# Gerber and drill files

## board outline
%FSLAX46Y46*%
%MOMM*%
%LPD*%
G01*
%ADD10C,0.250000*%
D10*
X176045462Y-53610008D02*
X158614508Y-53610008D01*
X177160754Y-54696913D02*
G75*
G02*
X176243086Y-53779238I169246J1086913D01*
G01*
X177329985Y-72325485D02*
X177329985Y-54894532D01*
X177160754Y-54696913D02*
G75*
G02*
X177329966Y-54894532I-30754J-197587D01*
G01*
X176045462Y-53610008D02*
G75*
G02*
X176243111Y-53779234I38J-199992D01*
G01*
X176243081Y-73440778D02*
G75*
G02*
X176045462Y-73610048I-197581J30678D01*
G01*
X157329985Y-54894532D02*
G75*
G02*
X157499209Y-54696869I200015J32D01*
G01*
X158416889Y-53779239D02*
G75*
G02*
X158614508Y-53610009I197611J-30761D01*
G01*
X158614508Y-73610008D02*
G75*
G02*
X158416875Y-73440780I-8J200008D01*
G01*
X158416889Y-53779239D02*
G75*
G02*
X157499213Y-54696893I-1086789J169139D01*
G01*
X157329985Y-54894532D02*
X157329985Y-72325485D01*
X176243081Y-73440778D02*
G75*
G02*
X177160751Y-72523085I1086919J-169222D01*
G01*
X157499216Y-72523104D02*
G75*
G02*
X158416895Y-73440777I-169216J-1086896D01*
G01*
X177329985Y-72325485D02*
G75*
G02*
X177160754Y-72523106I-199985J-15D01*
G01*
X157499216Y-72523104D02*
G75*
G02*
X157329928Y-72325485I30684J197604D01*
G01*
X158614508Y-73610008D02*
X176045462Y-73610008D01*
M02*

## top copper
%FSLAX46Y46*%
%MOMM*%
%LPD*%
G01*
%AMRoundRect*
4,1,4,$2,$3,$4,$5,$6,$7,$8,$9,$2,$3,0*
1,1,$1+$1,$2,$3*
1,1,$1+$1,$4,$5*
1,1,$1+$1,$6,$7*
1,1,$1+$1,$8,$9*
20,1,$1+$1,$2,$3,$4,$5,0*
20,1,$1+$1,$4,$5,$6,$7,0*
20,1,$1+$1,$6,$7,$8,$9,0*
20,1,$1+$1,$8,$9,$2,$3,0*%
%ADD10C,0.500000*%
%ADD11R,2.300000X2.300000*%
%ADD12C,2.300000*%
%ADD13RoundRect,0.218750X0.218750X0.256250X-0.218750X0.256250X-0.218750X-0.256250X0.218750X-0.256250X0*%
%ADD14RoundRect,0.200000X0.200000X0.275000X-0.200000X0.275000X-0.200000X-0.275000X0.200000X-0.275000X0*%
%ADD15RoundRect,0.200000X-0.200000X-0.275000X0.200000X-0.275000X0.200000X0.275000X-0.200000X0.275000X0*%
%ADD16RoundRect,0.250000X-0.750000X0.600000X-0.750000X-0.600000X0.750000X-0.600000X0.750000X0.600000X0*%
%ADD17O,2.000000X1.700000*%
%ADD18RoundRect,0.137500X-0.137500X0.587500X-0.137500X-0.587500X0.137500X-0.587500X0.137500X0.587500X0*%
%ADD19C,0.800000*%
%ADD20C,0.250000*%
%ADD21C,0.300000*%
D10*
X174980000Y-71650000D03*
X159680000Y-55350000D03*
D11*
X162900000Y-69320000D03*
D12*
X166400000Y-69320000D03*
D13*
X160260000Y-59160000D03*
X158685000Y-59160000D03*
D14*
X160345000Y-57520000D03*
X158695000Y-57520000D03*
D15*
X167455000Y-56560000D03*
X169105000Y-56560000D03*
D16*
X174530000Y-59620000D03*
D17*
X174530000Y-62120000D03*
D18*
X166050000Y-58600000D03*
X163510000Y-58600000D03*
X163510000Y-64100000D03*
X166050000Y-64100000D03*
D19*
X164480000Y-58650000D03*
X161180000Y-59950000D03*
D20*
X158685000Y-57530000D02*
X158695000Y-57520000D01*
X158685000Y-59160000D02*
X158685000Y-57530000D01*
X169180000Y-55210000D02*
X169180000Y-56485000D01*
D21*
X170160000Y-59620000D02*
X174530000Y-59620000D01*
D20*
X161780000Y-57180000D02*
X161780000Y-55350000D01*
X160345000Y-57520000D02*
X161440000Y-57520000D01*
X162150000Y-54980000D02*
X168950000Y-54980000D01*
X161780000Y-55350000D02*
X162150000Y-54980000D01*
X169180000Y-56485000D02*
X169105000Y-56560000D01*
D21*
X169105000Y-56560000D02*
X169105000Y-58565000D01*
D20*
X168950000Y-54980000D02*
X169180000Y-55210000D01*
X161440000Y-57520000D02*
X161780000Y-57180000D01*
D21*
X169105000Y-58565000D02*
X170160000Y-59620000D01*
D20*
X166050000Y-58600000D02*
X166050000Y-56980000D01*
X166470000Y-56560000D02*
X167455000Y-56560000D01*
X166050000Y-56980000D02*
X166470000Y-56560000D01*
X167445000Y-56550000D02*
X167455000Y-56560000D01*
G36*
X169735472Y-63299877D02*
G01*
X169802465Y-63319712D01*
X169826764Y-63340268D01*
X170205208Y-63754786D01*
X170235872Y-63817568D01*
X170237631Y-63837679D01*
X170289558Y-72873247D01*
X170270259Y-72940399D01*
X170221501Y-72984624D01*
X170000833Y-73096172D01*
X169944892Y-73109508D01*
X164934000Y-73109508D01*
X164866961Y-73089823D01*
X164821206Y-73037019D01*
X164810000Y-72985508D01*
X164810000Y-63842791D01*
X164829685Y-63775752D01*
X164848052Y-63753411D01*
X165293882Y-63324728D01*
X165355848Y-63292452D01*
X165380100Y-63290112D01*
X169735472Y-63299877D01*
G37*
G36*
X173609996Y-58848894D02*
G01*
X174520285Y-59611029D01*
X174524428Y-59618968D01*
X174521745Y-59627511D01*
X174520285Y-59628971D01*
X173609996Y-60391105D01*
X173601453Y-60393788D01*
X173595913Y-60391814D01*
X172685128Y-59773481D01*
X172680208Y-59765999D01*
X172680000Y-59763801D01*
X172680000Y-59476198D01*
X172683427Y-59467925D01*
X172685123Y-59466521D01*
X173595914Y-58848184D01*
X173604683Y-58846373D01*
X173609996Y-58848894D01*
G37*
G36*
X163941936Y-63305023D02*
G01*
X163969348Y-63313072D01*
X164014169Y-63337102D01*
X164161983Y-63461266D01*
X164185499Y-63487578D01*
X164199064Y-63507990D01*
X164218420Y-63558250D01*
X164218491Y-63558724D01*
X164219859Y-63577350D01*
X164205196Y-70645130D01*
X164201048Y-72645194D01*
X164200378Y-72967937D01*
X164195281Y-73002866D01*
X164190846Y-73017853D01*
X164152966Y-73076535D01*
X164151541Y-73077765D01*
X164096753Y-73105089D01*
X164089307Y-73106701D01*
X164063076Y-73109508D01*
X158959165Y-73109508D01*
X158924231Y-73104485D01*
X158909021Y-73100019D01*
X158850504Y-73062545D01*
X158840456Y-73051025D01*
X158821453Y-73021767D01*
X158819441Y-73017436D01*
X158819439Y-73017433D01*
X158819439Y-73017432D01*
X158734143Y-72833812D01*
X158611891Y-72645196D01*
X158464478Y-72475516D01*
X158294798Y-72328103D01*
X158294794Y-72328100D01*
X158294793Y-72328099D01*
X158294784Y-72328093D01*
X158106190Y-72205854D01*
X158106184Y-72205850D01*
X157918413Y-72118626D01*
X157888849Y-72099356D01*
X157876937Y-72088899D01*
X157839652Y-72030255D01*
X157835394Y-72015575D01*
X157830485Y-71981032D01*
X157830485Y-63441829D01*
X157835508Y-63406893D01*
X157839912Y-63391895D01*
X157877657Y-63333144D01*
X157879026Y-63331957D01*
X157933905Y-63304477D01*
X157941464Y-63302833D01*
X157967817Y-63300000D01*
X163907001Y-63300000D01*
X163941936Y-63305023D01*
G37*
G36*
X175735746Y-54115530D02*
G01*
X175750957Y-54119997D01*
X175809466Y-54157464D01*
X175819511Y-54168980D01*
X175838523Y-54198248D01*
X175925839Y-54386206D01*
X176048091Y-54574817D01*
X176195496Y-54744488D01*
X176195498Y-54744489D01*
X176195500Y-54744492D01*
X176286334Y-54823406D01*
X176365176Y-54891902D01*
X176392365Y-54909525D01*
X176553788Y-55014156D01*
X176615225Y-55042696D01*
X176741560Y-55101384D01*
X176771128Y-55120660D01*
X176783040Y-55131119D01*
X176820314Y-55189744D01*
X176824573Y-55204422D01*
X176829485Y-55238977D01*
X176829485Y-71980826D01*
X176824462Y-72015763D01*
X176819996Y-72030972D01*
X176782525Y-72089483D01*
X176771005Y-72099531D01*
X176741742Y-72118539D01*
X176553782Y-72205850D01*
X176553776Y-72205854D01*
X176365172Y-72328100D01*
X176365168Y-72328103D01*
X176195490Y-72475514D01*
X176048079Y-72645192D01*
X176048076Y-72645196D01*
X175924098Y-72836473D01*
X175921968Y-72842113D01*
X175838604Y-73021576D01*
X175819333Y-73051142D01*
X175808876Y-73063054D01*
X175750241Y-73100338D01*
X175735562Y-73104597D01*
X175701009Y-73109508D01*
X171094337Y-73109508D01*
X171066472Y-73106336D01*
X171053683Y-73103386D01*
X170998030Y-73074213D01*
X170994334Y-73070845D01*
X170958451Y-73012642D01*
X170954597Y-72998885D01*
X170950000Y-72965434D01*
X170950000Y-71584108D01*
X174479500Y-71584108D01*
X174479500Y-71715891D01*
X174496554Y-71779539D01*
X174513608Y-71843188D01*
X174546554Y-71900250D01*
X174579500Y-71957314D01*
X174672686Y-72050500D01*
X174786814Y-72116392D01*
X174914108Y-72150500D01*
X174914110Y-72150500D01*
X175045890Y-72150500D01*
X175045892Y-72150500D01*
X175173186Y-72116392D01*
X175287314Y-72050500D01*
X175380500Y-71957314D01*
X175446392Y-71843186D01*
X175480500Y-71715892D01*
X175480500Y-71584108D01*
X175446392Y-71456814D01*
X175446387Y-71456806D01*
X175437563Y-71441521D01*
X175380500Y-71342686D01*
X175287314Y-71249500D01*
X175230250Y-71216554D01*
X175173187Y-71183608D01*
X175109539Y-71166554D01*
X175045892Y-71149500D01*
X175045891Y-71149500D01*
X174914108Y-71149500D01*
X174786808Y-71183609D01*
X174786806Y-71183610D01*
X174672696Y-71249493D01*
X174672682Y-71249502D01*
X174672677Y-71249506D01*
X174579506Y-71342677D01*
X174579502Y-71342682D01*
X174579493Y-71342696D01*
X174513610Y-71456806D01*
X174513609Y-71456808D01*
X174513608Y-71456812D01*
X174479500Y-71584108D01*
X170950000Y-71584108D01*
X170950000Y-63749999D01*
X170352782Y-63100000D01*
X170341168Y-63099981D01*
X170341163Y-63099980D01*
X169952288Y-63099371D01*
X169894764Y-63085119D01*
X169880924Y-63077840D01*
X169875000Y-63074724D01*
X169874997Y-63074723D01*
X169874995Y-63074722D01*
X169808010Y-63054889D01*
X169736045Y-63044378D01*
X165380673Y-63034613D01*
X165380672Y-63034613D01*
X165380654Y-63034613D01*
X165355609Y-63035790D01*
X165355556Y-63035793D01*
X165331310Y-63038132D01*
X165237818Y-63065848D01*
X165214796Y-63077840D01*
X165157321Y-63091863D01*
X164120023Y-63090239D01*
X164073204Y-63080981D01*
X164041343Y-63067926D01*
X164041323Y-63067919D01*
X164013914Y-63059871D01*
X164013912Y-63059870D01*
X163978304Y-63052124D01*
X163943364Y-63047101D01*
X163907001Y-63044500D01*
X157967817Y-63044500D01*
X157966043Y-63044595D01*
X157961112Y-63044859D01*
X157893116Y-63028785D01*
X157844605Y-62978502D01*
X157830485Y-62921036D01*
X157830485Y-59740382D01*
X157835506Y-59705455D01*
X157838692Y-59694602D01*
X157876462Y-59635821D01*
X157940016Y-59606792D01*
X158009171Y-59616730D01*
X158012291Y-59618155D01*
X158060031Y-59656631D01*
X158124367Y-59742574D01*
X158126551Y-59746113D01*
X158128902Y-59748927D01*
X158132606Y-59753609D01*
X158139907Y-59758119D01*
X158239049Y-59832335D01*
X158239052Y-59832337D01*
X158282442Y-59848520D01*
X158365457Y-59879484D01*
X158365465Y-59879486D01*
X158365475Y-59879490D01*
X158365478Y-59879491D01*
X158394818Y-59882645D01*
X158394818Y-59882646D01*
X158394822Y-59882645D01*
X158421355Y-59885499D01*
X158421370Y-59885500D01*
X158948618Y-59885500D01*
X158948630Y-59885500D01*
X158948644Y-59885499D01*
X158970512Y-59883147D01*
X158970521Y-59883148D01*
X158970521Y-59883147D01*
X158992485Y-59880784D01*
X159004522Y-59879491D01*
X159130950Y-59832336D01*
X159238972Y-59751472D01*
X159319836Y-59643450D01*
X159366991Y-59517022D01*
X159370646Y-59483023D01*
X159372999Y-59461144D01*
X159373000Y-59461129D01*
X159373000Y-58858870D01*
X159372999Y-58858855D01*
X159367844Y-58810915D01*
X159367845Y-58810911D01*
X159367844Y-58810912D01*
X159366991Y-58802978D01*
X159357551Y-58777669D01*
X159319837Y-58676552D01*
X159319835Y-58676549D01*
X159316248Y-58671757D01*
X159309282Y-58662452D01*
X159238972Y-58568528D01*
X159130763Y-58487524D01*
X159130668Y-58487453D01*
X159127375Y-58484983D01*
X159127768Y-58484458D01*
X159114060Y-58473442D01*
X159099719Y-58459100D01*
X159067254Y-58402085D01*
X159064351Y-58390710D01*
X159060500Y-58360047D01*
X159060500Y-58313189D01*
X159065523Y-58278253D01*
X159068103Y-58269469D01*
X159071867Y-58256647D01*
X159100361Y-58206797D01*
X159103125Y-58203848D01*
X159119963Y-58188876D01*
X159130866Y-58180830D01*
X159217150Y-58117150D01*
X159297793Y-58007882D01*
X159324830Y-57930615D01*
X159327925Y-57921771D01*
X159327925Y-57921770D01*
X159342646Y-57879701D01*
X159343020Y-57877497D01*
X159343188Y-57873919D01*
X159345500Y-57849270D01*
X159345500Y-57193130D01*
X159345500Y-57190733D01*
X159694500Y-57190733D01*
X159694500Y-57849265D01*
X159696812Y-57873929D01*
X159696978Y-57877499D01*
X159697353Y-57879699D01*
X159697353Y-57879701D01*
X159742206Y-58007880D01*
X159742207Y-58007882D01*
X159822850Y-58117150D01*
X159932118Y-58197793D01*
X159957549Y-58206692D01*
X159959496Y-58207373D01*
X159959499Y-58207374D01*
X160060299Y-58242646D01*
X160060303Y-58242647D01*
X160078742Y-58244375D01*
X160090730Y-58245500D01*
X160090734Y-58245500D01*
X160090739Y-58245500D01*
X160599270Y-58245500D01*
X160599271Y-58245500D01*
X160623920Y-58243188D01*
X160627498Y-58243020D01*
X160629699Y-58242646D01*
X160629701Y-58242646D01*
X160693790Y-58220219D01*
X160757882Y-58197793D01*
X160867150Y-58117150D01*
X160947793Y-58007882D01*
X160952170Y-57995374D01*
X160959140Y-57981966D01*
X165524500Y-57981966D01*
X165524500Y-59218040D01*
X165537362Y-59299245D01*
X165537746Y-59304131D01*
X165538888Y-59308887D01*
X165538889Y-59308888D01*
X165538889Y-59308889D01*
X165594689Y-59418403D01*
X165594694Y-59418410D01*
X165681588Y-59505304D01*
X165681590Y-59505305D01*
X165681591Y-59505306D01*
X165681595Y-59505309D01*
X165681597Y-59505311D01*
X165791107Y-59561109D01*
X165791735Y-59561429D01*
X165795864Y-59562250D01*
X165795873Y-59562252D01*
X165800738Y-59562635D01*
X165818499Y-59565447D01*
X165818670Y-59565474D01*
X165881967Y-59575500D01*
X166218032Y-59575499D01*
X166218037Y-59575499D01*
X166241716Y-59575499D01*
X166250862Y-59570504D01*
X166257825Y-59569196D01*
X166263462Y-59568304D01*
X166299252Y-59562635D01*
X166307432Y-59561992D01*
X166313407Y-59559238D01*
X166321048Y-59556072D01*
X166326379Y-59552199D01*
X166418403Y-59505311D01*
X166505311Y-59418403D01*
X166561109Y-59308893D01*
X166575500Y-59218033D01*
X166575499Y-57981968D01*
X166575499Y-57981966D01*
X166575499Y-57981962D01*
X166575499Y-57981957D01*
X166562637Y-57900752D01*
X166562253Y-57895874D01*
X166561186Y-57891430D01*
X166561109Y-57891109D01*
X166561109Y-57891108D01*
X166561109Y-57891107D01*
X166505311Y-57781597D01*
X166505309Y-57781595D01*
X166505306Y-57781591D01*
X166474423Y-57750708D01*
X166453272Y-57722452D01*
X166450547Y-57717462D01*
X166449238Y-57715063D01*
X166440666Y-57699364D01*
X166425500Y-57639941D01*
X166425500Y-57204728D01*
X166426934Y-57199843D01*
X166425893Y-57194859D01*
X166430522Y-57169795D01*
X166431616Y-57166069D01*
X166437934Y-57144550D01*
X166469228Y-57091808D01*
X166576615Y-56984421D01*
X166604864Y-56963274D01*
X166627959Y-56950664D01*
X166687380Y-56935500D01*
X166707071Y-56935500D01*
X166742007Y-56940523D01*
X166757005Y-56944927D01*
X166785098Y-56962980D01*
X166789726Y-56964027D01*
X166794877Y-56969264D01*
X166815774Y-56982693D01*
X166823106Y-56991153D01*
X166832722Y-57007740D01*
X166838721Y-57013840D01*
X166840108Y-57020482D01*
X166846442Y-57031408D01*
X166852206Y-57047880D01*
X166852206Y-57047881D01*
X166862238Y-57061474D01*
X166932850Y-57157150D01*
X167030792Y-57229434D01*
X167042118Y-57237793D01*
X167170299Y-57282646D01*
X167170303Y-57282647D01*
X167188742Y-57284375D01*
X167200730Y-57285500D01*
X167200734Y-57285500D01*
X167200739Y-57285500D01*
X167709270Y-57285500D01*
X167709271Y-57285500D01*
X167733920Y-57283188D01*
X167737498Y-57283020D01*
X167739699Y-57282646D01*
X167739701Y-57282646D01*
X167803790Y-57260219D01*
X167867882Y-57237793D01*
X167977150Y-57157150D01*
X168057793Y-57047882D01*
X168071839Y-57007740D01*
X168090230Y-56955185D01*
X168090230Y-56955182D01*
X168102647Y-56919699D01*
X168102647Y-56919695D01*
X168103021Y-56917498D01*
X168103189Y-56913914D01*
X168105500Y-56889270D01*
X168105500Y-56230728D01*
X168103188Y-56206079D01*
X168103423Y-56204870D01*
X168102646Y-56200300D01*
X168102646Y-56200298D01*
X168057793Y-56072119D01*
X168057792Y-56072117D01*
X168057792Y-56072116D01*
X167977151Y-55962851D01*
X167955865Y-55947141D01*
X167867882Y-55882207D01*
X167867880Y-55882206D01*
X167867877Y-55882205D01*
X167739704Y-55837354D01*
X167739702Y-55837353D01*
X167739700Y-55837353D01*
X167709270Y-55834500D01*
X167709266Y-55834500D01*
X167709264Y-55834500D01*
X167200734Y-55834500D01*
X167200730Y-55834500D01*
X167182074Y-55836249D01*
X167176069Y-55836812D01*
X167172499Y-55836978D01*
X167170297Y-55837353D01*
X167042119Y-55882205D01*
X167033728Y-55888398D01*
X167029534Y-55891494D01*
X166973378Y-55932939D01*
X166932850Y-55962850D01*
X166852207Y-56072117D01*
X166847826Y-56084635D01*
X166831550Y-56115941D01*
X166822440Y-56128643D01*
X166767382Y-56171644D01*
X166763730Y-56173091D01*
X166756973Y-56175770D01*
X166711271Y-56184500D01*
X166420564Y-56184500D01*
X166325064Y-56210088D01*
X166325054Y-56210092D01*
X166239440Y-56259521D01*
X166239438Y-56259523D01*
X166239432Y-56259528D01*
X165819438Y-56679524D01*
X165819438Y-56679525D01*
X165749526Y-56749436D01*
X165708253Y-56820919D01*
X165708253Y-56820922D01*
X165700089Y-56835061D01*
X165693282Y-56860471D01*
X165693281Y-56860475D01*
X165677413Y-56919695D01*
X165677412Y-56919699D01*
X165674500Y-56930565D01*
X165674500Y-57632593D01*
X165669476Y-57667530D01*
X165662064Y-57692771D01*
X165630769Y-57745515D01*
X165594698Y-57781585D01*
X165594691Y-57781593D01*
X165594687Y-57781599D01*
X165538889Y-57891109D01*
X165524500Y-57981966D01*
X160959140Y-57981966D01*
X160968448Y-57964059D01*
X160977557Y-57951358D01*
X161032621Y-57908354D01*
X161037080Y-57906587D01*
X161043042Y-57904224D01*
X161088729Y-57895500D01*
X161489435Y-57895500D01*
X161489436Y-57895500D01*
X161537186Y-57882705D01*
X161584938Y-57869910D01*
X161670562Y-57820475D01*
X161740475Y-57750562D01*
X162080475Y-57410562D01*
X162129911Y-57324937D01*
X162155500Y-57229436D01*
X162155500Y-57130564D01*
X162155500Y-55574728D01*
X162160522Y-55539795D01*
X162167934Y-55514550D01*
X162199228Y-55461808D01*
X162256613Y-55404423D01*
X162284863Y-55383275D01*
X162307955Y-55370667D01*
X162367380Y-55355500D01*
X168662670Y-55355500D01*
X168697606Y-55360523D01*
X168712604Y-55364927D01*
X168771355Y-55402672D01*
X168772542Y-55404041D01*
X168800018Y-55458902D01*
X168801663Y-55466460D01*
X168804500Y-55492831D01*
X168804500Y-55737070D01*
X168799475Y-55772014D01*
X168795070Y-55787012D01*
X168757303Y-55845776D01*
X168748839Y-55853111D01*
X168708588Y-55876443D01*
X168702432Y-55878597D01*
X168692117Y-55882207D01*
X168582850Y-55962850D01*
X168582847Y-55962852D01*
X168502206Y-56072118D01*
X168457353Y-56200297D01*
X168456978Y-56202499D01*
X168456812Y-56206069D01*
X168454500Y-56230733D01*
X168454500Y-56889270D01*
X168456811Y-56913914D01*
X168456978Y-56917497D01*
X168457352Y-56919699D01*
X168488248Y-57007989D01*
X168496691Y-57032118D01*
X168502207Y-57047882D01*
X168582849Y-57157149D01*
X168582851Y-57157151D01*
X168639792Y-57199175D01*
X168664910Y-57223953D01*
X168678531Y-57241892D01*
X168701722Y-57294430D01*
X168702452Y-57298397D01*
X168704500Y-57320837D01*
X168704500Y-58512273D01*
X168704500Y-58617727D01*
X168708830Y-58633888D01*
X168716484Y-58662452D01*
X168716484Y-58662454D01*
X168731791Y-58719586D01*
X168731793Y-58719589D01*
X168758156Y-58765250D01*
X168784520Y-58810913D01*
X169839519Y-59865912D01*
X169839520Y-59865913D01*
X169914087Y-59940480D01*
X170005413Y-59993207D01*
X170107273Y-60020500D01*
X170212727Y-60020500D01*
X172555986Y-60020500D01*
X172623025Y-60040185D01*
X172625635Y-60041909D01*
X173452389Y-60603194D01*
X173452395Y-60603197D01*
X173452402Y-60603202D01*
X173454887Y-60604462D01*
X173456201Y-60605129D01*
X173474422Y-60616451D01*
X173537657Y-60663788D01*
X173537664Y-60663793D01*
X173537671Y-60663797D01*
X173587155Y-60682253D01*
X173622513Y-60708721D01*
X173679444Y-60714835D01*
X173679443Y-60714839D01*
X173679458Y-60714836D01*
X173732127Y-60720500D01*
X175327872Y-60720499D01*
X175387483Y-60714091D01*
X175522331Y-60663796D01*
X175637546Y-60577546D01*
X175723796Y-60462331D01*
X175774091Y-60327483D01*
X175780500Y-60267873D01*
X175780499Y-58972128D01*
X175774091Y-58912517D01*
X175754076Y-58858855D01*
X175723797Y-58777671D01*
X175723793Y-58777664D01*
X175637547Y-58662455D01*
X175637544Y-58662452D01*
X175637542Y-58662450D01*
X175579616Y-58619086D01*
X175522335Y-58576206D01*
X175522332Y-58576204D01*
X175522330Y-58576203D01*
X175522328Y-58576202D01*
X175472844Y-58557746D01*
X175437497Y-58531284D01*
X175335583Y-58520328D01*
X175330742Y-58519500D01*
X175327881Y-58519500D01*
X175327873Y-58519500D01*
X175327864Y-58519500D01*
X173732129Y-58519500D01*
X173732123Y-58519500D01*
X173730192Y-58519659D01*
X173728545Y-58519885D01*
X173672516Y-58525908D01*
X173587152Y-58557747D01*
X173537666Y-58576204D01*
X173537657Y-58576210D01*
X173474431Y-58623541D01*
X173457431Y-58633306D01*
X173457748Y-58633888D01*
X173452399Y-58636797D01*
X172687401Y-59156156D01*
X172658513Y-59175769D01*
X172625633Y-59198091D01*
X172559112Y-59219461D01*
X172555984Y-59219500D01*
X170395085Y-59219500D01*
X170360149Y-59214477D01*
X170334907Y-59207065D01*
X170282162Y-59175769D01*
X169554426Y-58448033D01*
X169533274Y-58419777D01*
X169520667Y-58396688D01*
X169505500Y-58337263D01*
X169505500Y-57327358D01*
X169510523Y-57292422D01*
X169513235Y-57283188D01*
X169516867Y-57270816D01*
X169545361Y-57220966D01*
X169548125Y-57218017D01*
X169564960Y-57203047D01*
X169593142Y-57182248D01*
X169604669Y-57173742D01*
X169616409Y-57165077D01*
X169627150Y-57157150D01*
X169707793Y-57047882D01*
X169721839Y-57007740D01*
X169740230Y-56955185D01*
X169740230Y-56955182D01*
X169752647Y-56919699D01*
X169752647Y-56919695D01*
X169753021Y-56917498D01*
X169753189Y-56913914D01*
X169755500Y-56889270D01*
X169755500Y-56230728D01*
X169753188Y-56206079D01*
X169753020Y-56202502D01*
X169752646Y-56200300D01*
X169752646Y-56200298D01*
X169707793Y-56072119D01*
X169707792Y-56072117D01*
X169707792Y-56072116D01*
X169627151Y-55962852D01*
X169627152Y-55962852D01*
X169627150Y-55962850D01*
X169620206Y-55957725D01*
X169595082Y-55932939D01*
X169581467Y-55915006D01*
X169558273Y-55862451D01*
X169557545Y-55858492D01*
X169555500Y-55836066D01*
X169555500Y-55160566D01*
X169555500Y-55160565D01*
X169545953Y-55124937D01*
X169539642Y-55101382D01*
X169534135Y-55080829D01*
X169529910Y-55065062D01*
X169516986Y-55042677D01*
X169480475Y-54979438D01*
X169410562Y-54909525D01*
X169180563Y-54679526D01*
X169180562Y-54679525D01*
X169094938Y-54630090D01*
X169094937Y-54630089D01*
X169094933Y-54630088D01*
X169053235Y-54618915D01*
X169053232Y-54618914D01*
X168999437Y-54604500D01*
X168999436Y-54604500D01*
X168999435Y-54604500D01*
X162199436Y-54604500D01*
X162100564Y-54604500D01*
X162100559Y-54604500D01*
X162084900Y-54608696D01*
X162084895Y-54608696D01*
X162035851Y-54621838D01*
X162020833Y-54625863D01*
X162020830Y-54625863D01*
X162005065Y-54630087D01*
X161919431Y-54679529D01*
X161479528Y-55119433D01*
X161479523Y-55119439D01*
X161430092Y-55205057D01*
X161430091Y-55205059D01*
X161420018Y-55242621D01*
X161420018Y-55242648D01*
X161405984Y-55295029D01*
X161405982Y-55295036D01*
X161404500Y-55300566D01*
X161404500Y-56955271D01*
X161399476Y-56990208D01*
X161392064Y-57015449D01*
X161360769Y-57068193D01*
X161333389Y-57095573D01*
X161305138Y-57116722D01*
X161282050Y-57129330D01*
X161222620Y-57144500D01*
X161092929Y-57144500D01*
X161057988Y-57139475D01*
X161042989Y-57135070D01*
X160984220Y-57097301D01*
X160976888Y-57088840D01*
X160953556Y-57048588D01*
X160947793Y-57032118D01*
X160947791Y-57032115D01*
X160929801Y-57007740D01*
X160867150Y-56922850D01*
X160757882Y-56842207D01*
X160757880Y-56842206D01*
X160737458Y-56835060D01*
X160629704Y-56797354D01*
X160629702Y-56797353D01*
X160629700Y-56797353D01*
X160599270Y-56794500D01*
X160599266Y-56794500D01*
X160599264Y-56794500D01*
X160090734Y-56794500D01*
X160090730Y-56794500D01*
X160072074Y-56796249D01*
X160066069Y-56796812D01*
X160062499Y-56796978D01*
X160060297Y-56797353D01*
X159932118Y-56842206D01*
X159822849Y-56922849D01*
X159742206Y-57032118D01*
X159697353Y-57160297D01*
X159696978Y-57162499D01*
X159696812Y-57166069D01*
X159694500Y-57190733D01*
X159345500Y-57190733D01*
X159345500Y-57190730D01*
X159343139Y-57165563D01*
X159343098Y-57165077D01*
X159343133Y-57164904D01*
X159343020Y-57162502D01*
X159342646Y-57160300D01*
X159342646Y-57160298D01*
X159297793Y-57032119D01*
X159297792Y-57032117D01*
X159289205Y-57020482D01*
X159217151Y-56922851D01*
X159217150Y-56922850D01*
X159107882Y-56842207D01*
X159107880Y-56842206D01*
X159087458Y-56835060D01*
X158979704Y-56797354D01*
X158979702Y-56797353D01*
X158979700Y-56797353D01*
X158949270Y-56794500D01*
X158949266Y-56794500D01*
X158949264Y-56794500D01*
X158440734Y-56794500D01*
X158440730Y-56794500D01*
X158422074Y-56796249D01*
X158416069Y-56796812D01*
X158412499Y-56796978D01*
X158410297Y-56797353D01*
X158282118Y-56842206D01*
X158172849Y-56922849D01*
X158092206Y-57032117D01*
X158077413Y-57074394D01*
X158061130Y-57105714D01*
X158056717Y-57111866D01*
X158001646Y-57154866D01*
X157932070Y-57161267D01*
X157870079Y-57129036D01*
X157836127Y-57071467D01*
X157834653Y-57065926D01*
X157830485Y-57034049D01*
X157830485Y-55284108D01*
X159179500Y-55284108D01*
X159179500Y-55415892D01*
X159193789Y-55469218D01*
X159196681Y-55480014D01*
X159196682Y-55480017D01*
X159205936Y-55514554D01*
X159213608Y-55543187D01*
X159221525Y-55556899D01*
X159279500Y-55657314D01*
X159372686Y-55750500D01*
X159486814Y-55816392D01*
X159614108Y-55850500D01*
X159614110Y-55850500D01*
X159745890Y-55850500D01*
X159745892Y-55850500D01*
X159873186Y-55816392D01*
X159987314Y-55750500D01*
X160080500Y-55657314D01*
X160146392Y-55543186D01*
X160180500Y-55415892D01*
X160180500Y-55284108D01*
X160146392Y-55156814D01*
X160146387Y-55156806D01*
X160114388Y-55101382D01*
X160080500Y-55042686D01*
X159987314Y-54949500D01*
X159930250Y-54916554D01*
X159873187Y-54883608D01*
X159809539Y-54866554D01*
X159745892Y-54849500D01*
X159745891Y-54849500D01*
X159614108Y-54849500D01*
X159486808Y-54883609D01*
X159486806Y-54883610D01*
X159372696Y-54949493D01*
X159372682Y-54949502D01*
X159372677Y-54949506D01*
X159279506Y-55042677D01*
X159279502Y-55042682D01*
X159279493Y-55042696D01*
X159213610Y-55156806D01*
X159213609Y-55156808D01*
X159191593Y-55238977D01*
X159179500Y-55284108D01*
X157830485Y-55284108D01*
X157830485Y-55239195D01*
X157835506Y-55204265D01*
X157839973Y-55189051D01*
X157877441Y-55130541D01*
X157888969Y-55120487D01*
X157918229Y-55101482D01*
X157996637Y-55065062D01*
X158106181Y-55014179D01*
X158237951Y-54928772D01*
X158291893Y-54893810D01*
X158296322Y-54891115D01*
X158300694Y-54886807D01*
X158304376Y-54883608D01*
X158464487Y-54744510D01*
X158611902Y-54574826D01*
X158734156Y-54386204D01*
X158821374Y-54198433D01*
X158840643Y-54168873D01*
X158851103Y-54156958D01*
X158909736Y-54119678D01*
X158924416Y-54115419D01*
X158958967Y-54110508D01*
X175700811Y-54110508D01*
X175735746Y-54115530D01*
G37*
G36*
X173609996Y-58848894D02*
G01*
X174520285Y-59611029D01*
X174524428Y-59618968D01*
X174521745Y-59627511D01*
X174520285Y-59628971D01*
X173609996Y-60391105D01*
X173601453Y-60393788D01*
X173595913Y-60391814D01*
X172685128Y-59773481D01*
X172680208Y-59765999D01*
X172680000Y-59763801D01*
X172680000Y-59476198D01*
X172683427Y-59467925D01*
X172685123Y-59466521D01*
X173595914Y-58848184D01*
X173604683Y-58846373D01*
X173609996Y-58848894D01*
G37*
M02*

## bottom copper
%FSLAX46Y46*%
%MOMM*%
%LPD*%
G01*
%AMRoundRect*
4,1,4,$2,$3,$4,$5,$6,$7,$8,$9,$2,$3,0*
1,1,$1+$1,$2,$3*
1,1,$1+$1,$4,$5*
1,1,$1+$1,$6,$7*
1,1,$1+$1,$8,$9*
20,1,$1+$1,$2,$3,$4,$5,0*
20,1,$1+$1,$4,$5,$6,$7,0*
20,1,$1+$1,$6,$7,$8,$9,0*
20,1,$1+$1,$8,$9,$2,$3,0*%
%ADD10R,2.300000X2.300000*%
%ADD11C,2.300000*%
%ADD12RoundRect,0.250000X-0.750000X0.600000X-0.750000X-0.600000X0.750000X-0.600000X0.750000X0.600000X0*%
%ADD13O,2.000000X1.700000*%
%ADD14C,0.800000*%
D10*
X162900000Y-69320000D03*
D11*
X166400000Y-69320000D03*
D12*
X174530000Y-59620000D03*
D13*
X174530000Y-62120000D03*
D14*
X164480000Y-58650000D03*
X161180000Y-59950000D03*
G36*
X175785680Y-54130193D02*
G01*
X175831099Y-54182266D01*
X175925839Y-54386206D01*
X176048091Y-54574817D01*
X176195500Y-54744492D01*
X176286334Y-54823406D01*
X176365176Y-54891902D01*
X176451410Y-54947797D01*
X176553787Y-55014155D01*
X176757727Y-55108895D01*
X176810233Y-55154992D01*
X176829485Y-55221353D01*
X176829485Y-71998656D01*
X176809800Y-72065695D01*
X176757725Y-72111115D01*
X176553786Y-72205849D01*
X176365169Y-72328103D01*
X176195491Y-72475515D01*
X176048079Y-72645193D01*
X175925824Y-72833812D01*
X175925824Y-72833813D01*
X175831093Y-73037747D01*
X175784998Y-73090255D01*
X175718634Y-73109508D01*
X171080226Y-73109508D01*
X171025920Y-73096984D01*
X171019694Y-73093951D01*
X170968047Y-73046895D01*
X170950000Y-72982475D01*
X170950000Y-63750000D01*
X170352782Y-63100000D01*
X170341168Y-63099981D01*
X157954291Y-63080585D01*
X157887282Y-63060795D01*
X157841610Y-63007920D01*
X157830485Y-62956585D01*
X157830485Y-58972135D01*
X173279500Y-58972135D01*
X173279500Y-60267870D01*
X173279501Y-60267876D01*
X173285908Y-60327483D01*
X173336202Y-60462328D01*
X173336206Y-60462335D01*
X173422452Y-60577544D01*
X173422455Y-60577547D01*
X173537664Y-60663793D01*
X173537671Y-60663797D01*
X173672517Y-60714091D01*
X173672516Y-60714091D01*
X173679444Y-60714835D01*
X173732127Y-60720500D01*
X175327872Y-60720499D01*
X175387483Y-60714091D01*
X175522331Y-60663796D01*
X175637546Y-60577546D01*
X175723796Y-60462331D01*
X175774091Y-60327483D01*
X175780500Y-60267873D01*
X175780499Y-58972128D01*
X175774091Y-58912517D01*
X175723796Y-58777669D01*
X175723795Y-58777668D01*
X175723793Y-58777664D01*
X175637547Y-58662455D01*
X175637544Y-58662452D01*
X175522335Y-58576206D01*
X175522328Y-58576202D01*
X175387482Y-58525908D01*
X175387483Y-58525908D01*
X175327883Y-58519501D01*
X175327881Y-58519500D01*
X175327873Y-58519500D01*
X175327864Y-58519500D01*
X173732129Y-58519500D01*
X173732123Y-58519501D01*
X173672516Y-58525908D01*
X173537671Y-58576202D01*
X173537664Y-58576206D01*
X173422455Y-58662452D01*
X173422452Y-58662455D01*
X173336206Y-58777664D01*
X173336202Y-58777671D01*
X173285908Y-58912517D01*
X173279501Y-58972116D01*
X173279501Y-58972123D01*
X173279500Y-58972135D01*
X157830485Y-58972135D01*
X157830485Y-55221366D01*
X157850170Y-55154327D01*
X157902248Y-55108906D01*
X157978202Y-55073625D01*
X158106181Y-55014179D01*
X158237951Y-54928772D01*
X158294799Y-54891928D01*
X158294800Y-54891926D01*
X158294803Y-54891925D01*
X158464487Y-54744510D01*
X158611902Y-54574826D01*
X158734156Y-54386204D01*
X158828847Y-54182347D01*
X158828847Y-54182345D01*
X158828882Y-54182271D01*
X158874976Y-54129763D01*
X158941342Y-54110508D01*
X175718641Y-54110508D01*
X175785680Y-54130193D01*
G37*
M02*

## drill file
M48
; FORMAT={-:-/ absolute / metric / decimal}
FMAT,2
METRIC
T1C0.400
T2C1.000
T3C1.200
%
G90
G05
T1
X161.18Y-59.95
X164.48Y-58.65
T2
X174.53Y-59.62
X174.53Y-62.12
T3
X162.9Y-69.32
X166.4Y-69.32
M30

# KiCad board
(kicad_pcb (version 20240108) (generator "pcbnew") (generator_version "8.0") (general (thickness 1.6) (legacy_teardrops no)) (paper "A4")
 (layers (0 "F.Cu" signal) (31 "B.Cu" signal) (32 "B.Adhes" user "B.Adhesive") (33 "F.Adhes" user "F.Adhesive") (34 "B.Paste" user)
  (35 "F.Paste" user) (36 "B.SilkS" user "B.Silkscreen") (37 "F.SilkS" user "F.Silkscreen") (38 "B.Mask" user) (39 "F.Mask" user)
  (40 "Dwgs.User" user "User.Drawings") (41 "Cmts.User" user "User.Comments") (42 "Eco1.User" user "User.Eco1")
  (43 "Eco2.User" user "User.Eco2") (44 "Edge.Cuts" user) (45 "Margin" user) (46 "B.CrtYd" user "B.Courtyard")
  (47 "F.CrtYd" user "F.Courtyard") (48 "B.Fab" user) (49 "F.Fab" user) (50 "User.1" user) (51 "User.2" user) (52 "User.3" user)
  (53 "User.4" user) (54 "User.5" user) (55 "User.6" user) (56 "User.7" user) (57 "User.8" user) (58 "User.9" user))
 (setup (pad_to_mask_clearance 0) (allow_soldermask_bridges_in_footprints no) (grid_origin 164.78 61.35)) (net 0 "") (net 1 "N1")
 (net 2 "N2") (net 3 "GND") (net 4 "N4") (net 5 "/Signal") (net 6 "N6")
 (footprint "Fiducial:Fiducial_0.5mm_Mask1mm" (layer "F.Cu") (at 174.98 71.65)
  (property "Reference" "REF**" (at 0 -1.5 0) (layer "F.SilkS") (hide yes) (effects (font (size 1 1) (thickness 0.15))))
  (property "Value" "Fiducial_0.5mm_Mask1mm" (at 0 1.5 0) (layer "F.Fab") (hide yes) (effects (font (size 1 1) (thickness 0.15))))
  (pad "" smd circle (at 0 0) (size 0.5 0.5) (layers "F.Cu" "F.Mask") (solder_mask_margin 0.25) (clearance 0.25)))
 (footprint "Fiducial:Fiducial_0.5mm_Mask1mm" (layer "F.Cu") (at 159.68 55.35)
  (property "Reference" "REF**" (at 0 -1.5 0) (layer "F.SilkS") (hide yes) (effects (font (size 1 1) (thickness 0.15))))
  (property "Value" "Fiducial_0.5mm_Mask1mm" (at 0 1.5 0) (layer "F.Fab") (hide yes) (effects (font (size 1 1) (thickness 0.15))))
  (pad "" smd circle (at 0 0) (size 0.5 0.5) (layers "F.Cu" "F.Mask") (solder_mask_margin 0.25) (clearance 0.25)))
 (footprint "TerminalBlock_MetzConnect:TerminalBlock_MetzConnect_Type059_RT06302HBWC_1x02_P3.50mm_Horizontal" (layer "F.Cu")
  (at 162.9 69.32)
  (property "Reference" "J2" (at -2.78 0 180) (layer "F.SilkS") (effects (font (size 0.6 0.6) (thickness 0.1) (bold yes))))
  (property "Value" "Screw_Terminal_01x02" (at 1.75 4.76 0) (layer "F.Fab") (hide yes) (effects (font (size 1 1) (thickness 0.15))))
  (pad "1" thru_hole rect (at 0 0) (size 2.3 2.3) (drill 1.2) (layers "*.Cu" "*.Mask") (remove_unused_layers no) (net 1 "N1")
   (teardrops (best_length_ratio 0.5) (max_length 1) (best_width_ratio 1) (max_width 2) (curve_points 0) (filter_ratio 0.9) (enabled yes)
    (allow_two_segments yes) (prefer_zone_connections yes)))
  (pad "2" thru_hole circle (at 3.5 0) (size 2.3 2.3) (drill 1.2) (layers "*.Cu" "*.Mask") (remove_unused_layers no) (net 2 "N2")
   (teardrops (best_length_ratio 0.5) (max_length 1) (best_width_ratio 1) (max_width 2) (curve_points 0) (filter_ratio 0.9) (enabled yes)
    (allow_two_segments yes) (prefer_zone_connections yes))))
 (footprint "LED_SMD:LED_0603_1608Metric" (layer "F.Cu") (at 159.4725 59.16 180)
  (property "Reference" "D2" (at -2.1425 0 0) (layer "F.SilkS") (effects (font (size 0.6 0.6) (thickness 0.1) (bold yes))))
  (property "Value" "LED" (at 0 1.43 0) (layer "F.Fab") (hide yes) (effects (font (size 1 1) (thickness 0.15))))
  (pad "1" smd roundrect (at -0.7875 0 180) (size 0.875 0.95) (layers "F.Cu" "F.Paste" "F.Mask") (roundrect_rratio 0.25) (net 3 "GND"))
  (pad "2" smd roundrect (at 0.7875 0 180) (size 0.875 0.95) (layers "F.Cu" "F.Paste" "F.Mask") (roundrect_rratio 0.25) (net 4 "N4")))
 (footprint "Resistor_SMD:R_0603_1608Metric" (layer "F.Cu") (at 159.52 57.52 180)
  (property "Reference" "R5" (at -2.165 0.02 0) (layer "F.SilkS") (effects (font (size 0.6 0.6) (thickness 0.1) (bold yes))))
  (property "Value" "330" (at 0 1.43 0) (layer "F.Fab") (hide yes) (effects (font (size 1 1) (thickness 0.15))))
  (pad "1" smd roundrect (at -0.825 0 180) (size 0.8 0.95) (layers "F.Cu" "F.Paste" "F.Mask") (roundrect_rratio 0.25) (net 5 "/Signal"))
  (pad "2" smd roundrect (at 0.825 0 180) (size 0.8 0.95) (layers "F.Cu" "F.Paste" "F.Mask") (roundrect_rratio 0.25) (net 4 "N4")))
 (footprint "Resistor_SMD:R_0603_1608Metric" (layer "F.Cu") (at 168.28 56.56)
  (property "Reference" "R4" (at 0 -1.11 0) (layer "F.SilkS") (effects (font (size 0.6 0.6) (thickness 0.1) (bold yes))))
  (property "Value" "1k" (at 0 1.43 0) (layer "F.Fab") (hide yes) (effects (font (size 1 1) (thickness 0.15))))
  (pad "1" smd roundrect (at -0.825 0) (size 0.8 0.95) (layers "F.Cu" "F.Paste" "F.Mask") (roundrect_rratio 0.25) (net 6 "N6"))
  (pad "2" smd roundrect (at 0.825 0) (size 0.8 0.95) (layers "F.Cu" "F.Paste" "F.Mask") (roundrect_rratio 0.25) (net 5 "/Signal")))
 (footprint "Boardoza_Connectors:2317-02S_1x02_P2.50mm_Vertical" (layer "F.Cu") (at 174.58 60.78 -90)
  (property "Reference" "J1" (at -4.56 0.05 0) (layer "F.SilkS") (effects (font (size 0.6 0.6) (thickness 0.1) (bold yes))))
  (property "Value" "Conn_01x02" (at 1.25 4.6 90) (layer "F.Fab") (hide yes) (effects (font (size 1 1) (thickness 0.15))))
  (pad "1" thru_hole roundrect (at -1.16 0.05 270) (size 1.7 2) (drill 1) (layers "*.Cu" "*.Mask") (remove_unused_layers no)
   (roundrect_rratio 0.1470588235) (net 5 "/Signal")
   (teardrops (best_length_ratio 0.5) (max_length 1) (best_width_ratio 1) (max_width 2) (curve_points 0) (filter_ratio 0.9) (enabled yes)
    (allow_two_segments yes) (prefer_zone_connections yes)))
  (pad "2" thru_hole oval (at 1.34 0.05 270) (size 1.7 2) (drill 1) (layers "*.Cu" "*.Mask") (remove_unused_layers no) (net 3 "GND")
   (teardrops (best_length_ratio 0.5) (max_length 1) (best_width_ratio 1) (max_width 2) (curve_points 0) (filter_ratio 0.9) (enabled yes)
    (allow_two_segments yes) (prefer_zone_connections yes))))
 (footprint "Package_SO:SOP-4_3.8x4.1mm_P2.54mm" (layer "F.Cu") (at 164.78 61.35 -90)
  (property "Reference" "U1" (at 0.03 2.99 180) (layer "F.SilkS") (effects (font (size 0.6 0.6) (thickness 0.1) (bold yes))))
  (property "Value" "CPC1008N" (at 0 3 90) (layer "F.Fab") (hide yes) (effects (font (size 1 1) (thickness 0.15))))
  (pad "1" smd roundrect (at -2.75 -1.27 270) (size 1.45 0.55) (layers "F.Cu" "F.Paste" "F.Mask") (roundrect_rratio 0.25) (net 6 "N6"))
  (pad "2" smd roundrect (at -2.75 1.27 270) (size 1.45 0.55) (layers "F.Cu" "F.Paste" "F.Mask") (roundrect_rratio 0.25) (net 3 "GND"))
  (pad "3" smd roundrect (at 2.75 1.27 270) (size 1.45 0.55) (layers "F.Cu" "F.Paste" "F.Mask") (roundrect_rratio 0.25) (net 1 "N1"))
  (pad "4" smd roundrect (at 2.75 -1.27 270) (size 1.45 0.55) (layers "F.Cu" "F.Paste" "F.Mask") (roundrect_rratio 0.25) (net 2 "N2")))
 (gr_line (start 176.045462 53.610008) (end 158.614508 53.610008) (stroke (width 0.25) (type solid)) (layer "Edge.Cuts"))
 (gr_arc (start 177.160754 54.696913) (mid 176.552172 54.387822) (end 176.243081 53.779239) (stroke (width 0.25) (type solid))
  (layer "Edge.Cuts"))
 (gr_line (start 177.329985 72.325485) (end 177.329985 54.894532) (stroke (width 0.25) (type solid)) (layer "Edge.Cuts"))
 (gr_arc (start 177.160754 54.696913) (mid 177.281894 54.764445) (end 177.329985 54.894532) (stroke (width 0.25) (type solid))
  (layer "Edge.Cuts"))
 (gr_arc (start 176.045462 53.610008) (mid 176.17555 53.658099) (end 176.243081 53.779239) (stroke (width 0.25) (type solid))
  (layer "Edge.Cuts"))
 (gr_arc (start 176.243081 73.440778) (mid 176.175561 73.561931) (end 176.045462 73.610008) (stroke (width 0.25) (type solid))
  (layer "Edge.Cuts"))
 (gr_arc (start 157.329985 54.894532) (mid 157.378074 54.764443) (end 157.499216 54.696913) (stroke (width 0.25) (type solid))
  (layer "Edge.Cuts"))
 (gr_arc (start 158.416889 53.779239) (mid 158.484418 53.658096) (end 158.614508 53.610008) (stroke (width 0.25) (type solid))
  (layer "Edge.Cuts"))
 (gr_arc (start 158.614508 73.610008) (mid 158.484415 73.561925) (end 158.416889 73.440778) (stroke (width 0.25) (type solid))
  (layer "Edge.Cuts"))
 (gr_arc (start 158.416889 53.779239) (mid 158.107816 54.38784) (end 157.499216 54.696913) (stroke (width 0.25) (type solid))
  (layer "Edge.Cuts"))
 (gr_line (start 157.329985 54.894532) (end 157.329985 72.325485) (stroke (width 0.25) (type solid)) (layer "Edge.Cuts"))
 (gr_arc (start 176.243081 73.440778) (mid 176.552162 72.832185) (end 177.160754 72.523104) (stroke (width 0.25) (type solid))
  (layer "Edge.Cuts"))
 (gr_arc (start 157.499216 72.523104) (mid 158.107807 72.832186) (end 158.416889 73.440778) (stroke (width 0.25) (type solid))
  (layer "Edge.Cuts"))
 (gr_arc (start 177.329985 72.325485) (mid 177.2819 72.455578) (end 177.160754 72.523104) (stroke (width 0.25) (type solid))
  (layer "Edge.Cuts"))
 (gr_arc (start 157.499216 72.523104) (mid 157.378059 72.455587) (end 157.329985 72.325485) (stroke (width 0.25) (type solid))
  (layer "Edge.Cuts"))
 (gr_line (start 158.614508 73.610008) (end 176.045462 73.610008) (stroke (width 0.25) (type solid)) (layer "Edge.Cuts"))
 (via (at 164.48 58.65) (size 0.8) (drill 0.4) (layers "F.Cu" "B.Cu") (free yes) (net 3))
 (via (at 161.18 59.95) (size 0.8) (drill 0.4) (layers "F.Cu" "B.Cu") (free yes) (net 3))
 (segment (start 158.685 57.53) (end 158.695 57.52) (width 0.25) (layer "F.Cu") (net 4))
 (segment (start 158.685 59.16) (end 158.685 57.53) (width 0.25) (layer "F.Cu") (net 4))
 (segment (start 169.18 55.21) (end 169.18 56.485) (width 0.25) (layer "F.Cu") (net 5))
 (segment (start 170.16 59.62) (end 174.53 59.62) (width 0.3) (layer "F.Cu") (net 5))
 (segment (start 161.78 57.18) (end 161.78 55.35) (width 0.25) (layer "F.Cu") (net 5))
 (segment (start 160.345 57.52) (end 161.44 57.52) (width 0.25) (layer "F.Cu") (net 5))
 (segment (start 162.15 54.98) (end 168.95 54.98) (width 0.25) (layer "F.Cu") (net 5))
 (segment (start 161.78 55.35) (end 162.15 54.98) (width 0.25) (layer "F.Cu") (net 5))
 (segment (start 169.18 56.485) (end 169.105 56.56) (width 0.25) (layer "F.Cu") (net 5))
 (segment (start 169.105 56.56) (end 169.105 58.565) (width 0.3) (layer "F.Cu") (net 5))
 (segment (start 168.95 54.98) (end 169.18 55.21) (width 0.25) (layer "F.Cu") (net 5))
 (segment (start 161.44 57.52) (end 161.78 57.18) (width 0.25) (layer "F.Cu") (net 5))
 (segment (start 169.105 58.565) (end 170.16 59.62) (width 0.3) (layer "F.Cu") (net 5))
 (segment (start 166.05 58.6) (end 166.05 56.98) (width 0.25) (layer "F.Cu") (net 6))
 (segment (start 166.47 56.56) (end 167.455 56.56) (width 0.25) (layer "F.Cu") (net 6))
 (segment (start 166.05 56.98) (end 166.47 56.56) (width 0.25) (layer "F.Cu") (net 6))
 (segment (start 167.445 56.55) (end 167.455 56.56) (width 0.25) (layer "F.Cu") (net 6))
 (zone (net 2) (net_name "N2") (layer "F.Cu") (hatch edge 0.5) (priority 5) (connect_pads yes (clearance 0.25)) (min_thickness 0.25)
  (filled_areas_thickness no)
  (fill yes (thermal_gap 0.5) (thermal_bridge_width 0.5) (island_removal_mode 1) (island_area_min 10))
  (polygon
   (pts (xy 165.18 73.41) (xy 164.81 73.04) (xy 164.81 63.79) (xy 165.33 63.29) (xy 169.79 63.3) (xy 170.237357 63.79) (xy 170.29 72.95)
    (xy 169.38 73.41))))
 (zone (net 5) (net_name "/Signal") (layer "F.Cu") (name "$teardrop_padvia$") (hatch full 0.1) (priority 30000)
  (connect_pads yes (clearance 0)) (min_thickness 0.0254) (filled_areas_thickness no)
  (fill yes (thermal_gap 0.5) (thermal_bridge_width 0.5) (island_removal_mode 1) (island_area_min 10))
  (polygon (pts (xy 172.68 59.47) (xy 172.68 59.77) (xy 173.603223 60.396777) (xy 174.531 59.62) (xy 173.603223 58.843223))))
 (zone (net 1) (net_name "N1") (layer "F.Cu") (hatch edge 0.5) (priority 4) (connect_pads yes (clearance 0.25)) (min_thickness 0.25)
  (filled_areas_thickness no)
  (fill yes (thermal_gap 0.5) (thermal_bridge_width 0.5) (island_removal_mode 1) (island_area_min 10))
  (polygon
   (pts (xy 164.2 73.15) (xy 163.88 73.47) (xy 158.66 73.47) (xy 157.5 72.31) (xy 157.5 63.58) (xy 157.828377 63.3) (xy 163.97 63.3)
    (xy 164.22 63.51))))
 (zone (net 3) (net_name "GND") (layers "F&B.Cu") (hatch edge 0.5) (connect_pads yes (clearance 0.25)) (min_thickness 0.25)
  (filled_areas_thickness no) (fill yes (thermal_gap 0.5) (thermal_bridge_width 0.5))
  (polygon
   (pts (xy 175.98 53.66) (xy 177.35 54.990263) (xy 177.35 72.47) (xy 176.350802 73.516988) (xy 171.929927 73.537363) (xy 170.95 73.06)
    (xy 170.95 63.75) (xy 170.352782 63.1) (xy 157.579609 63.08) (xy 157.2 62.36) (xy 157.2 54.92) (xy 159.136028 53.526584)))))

